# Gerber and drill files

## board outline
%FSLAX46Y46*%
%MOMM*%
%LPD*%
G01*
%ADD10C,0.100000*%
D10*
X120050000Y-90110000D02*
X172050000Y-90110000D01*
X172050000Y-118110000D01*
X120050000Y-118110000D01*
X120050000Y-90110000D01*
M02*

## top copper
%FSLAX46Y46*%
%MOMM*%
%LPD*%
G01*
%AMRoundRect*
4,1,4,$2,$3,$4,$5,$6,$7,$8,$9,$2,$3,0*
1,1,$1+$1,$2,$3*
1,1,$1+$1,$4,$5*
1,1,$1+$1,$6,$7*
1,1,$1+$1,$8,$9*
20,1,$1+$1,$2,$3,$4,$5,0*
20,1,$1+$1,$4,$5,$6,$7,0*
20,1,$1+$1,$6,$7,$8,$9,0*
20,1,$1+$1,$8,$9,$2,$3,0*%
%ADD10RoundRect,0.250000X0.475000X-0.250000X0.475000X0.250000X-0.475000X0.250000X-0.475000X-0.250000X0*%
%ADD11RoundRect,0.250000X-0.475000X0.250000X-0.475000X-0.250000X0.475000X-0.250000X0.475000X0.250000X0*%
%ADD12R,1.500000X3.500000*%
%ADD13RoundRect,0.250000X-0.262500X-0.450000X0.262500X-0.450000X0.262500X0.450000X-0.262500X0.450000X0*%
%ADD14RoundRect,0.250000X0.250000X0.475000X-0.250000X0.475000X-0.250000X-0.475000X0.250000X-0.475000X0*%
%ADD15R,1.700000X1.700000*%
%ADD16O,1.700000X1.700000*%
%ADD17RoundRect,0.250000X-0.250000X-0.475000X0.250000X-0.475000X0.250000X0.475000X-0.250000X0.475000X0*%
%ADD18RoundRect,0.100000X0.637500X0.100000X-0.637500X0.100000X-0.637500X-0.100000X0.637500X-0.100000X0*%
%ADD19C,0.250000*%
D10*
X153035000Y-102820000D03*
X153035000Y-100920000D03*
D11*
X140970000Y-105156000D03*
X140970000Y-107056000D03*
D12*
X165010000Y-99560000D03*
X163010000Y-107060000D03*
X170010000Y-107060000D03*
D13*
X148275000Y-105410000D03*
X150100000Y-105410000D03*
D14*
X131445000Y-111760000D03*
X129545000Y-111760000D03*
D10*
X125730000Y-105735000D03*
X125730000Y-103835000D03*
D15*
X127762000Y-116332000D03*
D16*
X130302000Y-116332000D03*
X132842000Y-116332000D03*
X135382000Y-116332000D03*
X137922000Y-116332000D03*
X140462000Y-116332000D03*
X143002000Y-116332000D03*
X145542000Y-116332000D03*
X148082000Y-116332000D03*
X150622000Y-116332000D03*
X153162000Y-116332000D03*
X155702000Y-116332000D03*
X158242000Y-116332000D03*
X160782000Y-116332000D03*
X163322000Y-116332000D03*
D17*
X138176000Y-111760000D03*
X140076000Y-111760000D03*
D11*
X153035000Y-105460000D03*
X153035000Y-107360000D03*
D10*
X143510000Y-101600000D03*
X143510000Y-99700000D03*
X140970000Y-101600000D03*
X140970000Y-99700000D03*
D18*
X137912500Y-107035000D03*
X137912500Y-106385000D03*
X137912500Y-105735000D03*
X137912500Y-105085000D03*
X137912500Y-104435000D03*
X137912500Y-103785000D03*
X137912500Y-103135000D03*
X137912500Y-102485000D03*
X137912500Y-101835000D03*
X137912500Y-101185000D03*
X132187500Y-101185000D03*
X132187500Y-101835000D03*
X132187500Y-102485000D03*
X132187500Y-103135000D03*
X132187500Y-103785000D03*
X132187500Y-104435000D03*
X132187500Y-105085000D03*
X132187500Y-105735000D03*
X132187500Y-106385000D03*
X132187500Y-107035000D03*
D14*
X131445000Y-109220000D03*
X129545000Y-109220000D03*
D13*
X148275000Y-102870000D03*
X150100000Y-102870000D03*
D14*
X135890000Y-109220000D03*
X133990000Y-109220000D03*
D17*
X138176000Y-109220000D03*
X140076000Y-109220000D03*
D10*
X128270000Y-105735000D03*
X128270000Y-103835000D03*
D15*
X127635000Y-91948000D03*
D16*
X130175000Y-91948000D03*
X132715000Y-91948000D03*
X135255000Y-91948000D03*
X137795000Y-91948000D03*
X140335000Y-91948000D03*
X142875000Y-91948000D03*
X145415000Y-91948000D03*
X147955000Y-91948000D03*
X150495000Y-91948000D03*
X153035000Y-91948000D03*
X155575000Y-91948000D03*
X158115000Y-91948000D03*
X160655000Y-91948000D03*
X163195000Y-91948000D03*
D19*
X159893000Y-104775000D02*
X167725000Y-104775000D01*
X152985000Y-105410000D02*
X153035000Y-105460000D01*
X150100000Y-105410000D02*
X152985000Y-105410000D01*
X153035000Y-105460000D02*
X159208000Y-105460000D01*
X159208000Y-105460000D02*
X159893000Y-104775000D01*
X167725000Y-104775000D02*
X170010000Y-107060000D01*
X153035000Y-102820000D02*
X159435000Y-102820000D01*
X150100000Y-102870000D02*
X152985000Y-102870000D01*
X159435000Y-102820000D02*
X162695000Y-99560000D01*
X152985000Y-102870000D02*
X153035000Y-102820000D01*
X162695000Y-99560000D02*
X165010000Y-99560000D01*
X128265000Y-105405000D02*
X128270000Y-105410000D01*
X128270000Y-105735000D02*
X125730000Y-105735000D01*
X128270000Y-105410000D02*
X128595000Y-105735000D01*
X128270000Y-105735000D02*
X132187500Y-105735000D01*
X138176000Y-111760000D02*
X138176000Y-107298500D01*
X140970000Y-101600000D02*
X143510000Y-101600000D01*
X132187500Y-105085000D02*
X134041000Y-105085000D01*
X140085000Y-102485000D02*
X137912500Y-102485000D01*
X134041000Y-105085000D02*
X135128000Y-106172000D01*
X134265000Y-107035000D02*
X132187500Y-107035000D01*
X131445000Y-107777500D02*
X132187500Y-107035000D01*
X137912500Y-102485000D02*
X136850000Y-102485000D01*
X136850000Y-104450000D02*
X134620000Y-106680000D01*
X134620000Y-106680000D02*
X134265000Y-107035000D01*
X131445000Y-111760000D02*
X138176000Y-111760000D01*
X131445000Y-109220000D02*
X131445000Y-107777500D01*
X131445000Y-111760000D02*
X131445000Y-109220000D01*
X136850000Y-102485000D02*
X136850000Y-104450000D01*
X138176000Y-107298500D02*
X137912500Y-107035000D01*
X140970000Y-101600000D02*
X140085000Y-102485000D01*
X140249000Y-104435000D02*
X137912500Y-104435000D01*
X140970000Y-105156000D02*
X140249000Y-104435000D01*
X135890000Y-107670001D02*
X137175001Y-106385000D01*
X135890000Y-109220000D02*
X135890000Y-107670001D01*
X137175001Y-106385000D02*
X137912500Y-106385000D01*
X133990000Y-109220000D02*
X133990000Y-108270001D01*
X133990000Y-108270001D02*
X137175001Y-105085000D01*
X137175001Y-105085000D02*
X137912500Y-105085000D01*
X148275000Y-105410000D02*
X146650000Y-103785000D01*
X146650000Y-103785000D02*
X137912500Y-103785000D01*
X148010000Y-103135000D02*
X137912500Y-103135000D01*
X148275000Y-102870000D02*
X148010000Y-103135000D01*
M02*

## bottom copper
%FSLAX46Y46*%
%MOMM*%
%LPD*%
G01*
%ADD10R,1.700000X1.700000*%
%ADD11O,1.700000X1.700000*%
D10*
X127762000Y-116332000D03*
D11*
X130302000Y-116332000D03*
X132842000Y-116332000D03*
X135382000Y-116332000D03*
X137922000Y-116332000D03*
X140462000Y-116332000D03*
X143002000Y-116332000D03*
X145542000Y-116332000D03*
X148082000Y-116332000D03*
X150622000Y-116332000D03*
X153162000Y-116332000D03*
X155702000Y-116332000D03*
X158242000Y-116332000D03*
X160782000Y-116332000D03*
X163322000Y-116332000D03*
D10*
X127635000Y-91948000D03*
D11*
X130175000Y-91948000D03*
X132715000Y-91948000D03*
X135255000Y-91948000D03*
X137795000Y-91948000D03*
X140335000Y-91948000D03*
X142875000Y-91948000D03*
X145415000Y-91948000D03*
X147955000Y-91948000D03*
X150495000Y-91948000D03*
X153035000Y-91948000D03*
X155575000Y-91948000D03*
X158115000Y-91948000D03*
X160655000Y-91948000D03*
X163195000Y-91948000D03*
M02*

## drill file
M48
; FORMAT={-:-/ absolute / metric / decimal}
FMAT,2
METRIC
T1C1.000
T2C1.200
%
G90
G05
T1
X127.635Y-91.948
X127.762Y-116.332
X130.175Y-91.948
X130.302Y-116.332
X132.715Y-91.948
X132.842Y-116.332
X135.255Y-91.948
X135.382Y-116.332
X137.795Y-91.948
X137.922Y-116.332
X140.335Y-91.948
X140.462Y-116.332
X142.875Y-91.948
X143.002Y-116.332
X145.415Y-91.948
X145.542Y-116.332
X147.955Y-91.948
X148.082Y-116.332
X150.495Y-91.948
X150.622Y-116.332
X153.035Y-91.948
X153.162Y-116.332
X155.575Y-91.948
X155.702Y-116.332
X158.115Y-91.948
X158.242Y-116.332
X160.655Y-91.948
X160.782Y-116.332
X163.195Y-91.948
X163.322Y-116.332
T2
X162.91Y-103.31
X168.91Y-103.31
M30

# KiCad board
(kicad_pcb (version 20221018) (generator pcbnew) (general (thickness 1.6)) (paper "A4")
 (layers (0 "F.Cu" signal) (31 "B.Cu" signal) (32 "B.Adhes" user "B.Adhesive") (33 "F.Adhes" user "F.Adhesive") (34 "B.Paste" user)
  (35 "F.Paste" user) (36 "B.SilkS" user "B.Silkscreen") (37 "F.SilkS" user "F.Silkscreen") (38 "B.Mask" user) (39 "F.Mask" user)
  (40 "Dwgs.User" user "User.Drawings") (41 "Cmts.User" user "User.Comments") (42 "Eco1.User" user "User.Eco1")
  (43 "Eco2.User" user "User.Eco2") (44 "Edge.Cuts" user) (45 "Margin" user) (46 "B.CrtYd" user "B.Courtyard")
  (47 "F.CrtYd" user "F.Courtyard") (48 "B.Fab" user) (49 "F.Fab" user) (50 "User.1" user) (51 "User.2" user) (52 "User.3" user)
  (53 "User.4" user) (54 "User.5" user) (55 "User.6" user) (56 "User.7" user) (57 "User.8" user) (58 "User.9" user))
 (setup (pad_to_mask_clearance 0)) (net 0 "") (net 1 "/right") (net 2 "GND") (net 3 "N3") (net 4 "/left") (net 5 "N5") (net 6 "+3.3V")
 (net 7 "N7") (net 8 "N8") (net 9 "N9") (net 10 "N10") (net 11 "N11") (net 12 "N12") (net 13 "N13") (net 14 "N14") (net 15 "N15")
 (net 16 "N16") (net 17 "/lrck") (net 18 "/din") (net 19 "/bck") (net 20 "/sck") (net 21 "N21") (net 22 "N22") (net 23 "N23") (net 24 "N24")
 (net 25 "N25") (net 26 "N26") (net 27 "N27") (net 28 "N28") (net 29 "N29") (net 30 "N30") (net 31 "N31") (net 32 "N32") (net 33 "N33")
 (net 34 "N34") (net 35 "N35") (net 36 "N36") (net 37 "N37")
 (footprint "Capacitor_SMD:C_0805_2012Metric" (layer "F.Cu") (at 153.035 101.87 90)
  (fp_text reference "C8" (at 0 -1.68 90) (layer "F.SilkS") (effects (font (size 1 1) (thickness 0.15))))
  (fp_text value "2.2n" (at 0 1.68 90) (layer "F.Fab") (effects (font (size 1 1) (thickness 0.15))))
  (pad "1" smd roundrect (at -0.95 0 90) (size 1 1.45) (layers "F.Cu" "F.Paste" "F.Mask") (roundrect_rratio 0.25) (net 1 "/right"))
  (pad "2" smd roundrect (at 0.95 0 90) (size 1 1.45) (layers "F.Cu" "F.Paste" "F.Mask") (roundrect_rratio 0.25) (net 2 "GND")))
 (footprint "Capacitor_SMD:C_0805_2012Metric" (layer "F.Cu") (at 140.97 106.106 -90)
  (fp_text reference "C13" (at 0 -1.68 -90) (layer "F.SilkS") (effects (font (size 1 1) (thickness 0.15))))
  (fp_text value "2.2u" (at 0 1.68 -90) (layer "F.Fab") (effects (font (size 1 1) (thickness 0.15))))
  (pad "1" smd roundrect (at -0.95 0 270) (size 1 1.45) (layers "F.Cu" "F.Paste" "F.Mask") (roundrect_rratio 0.25) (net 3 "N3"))
  (pad "2" smd roundrect (at 0.95 0 270) (size 1 1.45) (layers "F.Cu" "F.Paste" "F.Mask") (roundrect_rratio 0.25) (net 2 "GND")))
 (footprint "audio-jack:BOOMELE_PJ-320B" (layer "F.Cu") (at 165.91 103.31)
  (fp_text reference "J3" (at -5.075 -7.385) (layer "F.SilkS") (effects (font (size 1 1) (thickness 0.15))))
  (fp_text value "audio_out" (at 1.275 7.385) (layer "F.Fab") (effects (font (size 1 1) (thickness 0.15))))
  (pad "" np_thru_hole circle (at -3 0) (size 1.2 1.2) (drill 1.2) (layers "*.Cu" "*.Mask"))
  (pad "" np_thru_hole circle (at 3 0) (size 1.2 1.2) (drill 1.2) (layers "*.Cu" "*.Mask"))
  (pad "R" smd rect (at -0.9 -3.75) (size 1.5 3.5) (layers "F.Cu" "F.Paste" "F.Mask") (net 1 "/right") (solder_mask_margin 0.102))
  (pad "S" smd rect (at -2.9 3.75) (size 1.5 3.5) (layers "F.Cu" "F.Paste" "F.Mask") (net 2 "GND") (solder_mask_margin 0.102))
  (pad "T" smd rect (at 4.1 3.75) (size 1.5 3.5) (layers "F.Cu" "F.Paste" "F.Mask") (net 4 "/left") (solder_mask_margin 0.102)))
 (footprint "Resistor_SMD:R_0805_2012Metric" (layer "F.Cu") (at 149.1875 105.41)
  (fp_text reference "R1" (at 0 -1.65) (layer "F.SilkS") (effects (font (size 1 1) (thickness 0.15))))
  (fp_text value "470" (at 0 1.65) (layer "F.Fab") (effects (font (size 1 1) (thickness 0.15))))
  (pad "1" smd roundrect (at -0.9125 0) (size 1.025 1.4) (layers "F.Cu" "F.Paste" "F.Mask") (roundrect_rratio 0.243902) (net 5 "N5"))
  (pad "2" smd roundrect (at 0.9125 0) (size 1.025 1.4) (layers "F.Cu" "F.Paste" "F.Mask") (roundrect_rratio 0.243902) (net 4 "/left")))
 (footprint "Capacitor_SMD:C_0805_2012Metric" (layer "F.Cu") (at 130.495 111.76 180)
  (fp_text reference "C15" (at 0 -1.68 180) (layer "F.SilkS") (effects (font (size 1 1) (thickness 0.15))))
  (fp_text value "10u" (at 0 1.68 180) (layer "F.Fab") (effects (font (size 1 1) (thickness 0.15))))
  (pad "1" smd roundrect (at -0.95 0 180) (size 1 1.45) (layers "F.Cu" "F.Paste" "F.Mask") (roundrect_rratio 0.25) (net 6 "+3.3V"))
  (pad "2" smd roundrect (at 0.95 0 180) (size 1 1.45) (layers "F.Cu" "F.Paste" "F.Mask") (roundrect_rratio 0.25) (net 2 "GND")))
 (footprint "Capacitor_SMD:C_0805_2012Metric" (layer "F.Cu") (at 125.73 104.785 90)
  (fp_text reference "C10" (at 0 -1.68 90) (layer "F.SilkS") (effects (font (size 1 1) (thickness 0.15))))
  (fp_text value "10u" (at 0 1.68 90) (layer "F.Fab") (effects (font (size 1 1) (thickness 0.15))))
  (pad "1" smd roundrect (at -0.95 0 90) (size 1 1.45) (layers "F.Cu" "F.Paste" "F.Mask") (roundrect_rratio 0.25) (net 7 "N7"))
  (pad "2" smd roundrect (at 0.95 0 90) (size 1 1.45) (layers "F.Cu" "F.Paste" "F.Mask") (roundrect_rratio 0.25) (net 2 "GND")))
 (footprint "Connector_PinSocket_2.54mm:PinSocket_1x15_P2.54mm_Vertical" (layer "F.Cu") (at 127.762 116.332 90)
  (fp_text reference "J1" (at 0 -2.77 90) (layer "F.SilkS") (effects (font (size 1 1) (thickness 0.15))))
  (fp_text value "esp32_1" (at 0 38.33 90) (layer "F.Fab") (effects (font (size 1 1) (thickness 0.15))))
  (pad "1" thru_hole rect (at 0 0 90) (size 1.7 1.7) (drill 1) (layers "*.Cu" "*.Mask") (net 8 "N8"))
  (pad "2" thru_hole oval (at 0 2.54 90) (size 1.7 1.7) (drill 1) (layers "*.Cu" "*.Mask") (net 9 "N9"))
  (pad "3" thru_hole oval (at 0 5.08 90) (size 1.7 1.7) (drill 1) (layers "*.Cu" "*.Mask") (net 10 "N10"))
  (pad "4" thru_hole oval (at 0 7.62 90) (size 1.7 1.7) (drill 1) (layers "*.Cu" "*.Mask") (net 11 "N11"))
  (pad "5" thru_hole oval (at 0 10.16 90) (size 1.7 1.7) (drill 1) (layers "*.Cu" "*.Mask") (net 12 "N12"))
  (pad "6" thru_hole oval (at 0 12.7 90) (size 1.7 1.7) (drill 1) (layers "*.Cu" "*.Mask") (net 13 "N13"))
  (pad "7" thru_hole oval (at 0 15.24 90) (size 1.7 1.7) (drill 1) (layers "*.Cu" "*.Mask") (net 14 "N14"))
  (pad "8" thru_hole oval (at 0 17.78 90) (size 1.7 1.7) (drill 1) (layers "*.Cu" "*.Mask") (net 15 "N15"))
  (pad "9" thru_hole oval (at 0 20.32 90) (size 1.7 1.7) (drill 1) (layers "*.Cu" "*.Mask") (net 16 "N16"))
  (pad "10" thru_hole oval (at 0 22.86 90) (size 1.7 1.7) (drill 1) (layers "*.Cu" "*.Mask") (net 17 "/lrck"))
  (pad "11" thru_hole oval (at 0 25.4 90) (size 1.7 1.7) (drill 1) (layers "*.Cu" "*.Mask") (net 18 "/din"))
  (pad "12" thru_hole oval (at 0 27.94 90) (size 1.7 1.7) (drill 1) (layers "*.Cu" "*.Mask") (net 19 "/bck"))
  (pad "13" thru_hole oval (at 0 30.48 90) (size 1.7 1.7) (drill 1) (layers "*.Cu" "*.Mask") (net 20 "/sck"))
  (pad "14" thru_hole oval (at 0 33.02 90) (size 1.7 1.7) (drill 1) (layers "*.Cu" "*.Mask") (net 2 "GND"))
  (pad "15" thru_hole oval (at 0 35.56 90) (size 1.7 1.7) (drill 1) (layers "*.Cu" "*.Mask") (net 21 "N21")))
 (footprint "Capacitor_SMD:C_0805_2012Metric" (layer "F.Cu") (at 139.126 111.76)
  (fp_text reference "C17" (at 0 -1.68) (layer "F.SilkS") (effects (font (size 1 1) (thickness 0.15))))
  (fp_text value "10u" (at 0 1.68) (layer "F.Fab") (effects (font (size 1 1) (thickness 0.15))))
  (pad "1" smd roundrect (at -0.95 0) (size 1 1.45) (layers "F.Cu" "F.Paste" "F.Mask") (roundrect_rratio 0.25) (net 6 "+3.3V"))
  (pad "2" smd roundrect (at 0.95 0) (size 1 1.45) (layers "F.Cu" "F.Paste" "F.Mask") (roundrect_rratio 0.25) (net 2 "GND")))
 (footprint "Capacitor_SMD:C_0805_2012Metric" (layer "F.Cu") (at 153.035 106.41 -90)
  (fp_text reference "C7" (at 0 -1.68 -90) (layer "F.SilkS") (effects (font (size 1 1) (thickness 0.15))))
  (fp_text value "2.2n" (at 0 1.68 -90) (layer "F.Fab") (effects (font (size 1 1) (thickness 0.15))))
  (pad "1" smd roundrect (at -0.95 0 270) (size 1 1.45) (layers "F.Cu" "F.Paste" "F.Mask") (roundrect_rratio 0.25) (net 4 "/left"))
  (pad "2" smd roundrect (at 0.95 0 270) (size 1 1.45) (layers "F.Cu" "F.Paste" "F.Mask") (roundrect_rratio 0.25) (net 2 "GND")))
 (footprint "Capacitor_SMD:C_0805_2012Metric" (layer "F.Cu") (at 143.51 100.65 90)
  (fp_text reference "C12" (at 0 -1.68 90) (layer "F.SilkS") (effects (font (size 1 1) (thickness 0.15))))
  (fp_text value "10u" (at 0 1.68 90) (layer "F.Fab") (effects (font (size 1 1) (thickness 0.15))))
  (pad "1" smd roundrect (at -0.95 0 90) (size 1 1.45) (layers "F.Cu" "F.Paste" "F.Mask") (roundrect_rratio 0.25) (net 6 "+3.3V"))
  (pad "2" smd roundrect (at 0.95 0 90) (size 1 1.45) (layers "F.Cu" "F.Paste" "F.Mask") (roundrect_rratio 0.25) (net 2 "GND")))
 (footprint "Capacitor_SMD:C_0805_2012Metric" (layer "F.Cu") (at 140.97 100.65 90)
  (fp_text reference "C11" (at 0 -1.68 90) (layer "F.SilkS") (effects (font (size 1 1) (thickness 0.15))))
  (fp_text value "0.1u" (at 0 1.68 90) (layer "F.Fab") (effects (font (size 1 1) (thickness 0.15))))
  (pad "1" smd roundrect (at -0.95 0 90) (size 1 1.45) (layers "F.Cu" "F.Paste" "F.Mask") (roundrect_rratio 0.25) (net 6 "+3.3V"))
  (pad "2" smd roundrect (at 0.95 0 90) (size 1 1.45) (layers "F.Cu" "F.Paste" "F.Mask") (roundrect_rratio 0.25) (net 2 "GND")))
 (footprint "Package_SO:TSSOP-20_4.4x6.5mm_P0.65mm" (layer "F.Cu") (at 135.05 104.11 180)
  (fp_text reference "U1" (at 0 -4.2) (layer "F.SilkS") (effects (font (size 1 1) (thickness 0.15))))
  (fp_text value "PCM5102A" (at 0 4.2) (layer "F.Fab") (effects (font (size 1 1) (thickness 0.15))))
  (pad "1" smd roundrect (at -2.8625 -2.925 180) (size 1.475 0.4) (layers "F.Cu" "F.Paste" "F.Mask") (roundrect_rratio 0.25) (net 6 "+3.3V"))
  (pad "2" smd roundrect (at -2.8625 -2.275 180) (size 1.475 0.4) (layers "F.Cu" "F.Paste" "F.Mask") (roundrect_rratio 0.25) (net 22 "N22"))
  (pad "3" smd roundrect (at -2.8625 -1.625 180) (size 1.475 0.4) (layers "F.Cu" "F.Paste" "F.Mask") (roundrect_rratio 0.25) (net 2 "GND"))
  (pad "4" smd roundrect (at -2.8625 -0.975 180) (size 1.475 0.4) (layers "F.Cu" "F.Paste" "F.Mask") (roundrect_rratio 0.25) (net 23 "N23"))
  (pad "5" smd roundrect (at -2.8625 -0.325 180) (size 1.475 0.4) (layers "F.Cu" "F.Paste" "F.Mask") (roundrect_rratio 0.25) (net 3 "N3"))
  (pad "6" smd roundrect (at -2.8625 0.325 180) (size 1.475 0.4) (layers "F.Cu" "F.Paste" "F.Mask") (roundrect_rratio 0.25) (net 5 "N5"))
  (pad "7" smd roundrect (at -2.8625 0.975 180) (size 1.475 0.4) (layers "F.Cu" "F.Paste" "F.Mask") (roundrect_rratio 0.25) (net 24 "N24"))
  (pad "8" smd roundrect (at -2.8625 1.625 180) (size 1.475 0.4) (layers "F.Cu" "F.Paste" "F.Mask") (roundrect_rratio 0.25) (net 6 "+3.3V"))
  (pad "9" smd roundrect (at -2.8625 2.275 180) (size 1.475 0.4) (layers "F.Cu" "F.Paste" "F.Mask") (roundrect_rratio 0.25) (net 2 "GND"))
  (pad "10" smd roundrect (at -2.8625 2.925 180) (size 1.475 0.4) (layers "F.Cu" "F.Paste" "F.Mask") (roundrect_rratio 0.25) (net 2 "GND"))
  (pad "11" smd roundrect (at 2.8625 2.925 180) (size 1.475 0.4) (layers "F.Cu" "F.Paste" "F.Mask") (roundrect_rratio 0.25) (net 2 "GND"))
  (pad "12" smd roundrect (at 2.8625 2.275 180) (size 1.475 0.4) (layers "F.Cu" "F.Paste" "F.Mask") (roundrect_rratio 0.25) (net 20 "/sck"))
  (pad "13" smd roundrect (at 2.8625 1.625 180) (size 1.475 0.4) (layers "F.Cu" "F.Paste" "F.Mask") (roundrect_rratio 0.25) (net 19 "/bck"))
  (pad "14" smd roundrect (at 2.8625 0.975 180) (size 1.475 0.4) (layers "F.Cu" "F.Paste" "F.Mask") (roundrect_rratio 0.25) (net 18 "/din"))
  (pad "15" smd roundrect (at 2.8625 0.325 180) (size 1.475 0.4) (layers "F.Cu" "F.Paste" "F.Mask") (roundrect_rratio 0.25) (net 17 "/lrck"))
  (pad "16" smd roundrect (at 2.8625 -0.325 180) (size 1.475 0.4) (layers "F.Cu" "F.Paste" "F.Mask") (roundrect_rratio 0.25) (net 2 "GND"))
  (pad "17" smd roundrect (at 2.8625 -0.975 180) (size 1.475 0.4) (layers "F.Cu" "F.Paste" "F.Mask") (roundrect_rratio 0.25) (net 6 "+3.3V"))
  (pad "18" smd roundrect (at 2.8625 -1.625 180) (size 1.475 0.4) (layers "F.Cu" "F.Paste" "F.Mask") (roundrect_rratio 0.25) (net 7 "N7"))
  (pad "19" smd roundrect (at 2.8625 -2.275 180) (size 1.475 0.4) (layers "F.Cu" "F.Paste" "F.Mask") (roundrect_rratio 0.25) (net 2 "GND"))
  (pad "20" smd roundrect (at 2.8625 -2.925 180) (size 1.475 0.4) (layers "F.Cu" "F.Paste" "F.Mask") (roundrect_rratio 0.25) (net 6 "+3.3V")))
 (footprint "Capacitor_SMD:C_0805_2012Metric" (layer "F.Cu") (at 130.495 109.22 180)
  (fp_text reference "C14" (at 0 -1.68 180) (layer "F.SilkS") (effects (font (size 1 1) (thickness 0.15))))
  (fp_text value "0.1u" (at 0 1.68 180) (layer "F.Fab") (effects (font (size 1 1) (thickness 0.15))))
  (pad "1" smd roundrect (at -0.95 0 180) (size 1 1.45) (layers "F.Cu" "F.Paste" "F.Mask") (roundrect_rratio 0.25) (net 6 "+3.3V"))
  (pad "2" smd roundrect (at 0.95 0 180) (size 1 1.45) (layers "F.Cu" "F.Paste" "F.Mask") (roundrect_rratio 0.25) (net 2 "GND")))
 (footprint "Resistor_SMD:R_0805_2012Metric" (layer "F.Cu") (at 149.1875 102.87)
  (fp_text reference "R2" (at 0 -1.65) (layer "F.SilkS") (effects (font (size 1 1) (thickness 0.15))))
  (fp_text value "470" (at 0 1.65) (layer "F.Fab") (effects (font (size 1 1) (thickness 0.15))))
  (pad "1" smd roundrect (at -0.9125 0) (size 1.025 1.4) (layers "F.Cu" "F.Paste" "F.Mask") (roundrect_rratio 0.243902) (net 24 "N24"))
  (pad "2" smd roundrect (at 0.9125 0) (size 1.025 1.4) (layers "F.Cu" "F.Paste" "F.Mask") (roundrect_rratio 0.243902) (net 1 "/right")))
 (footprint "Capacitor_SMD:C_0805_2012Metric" (layer "F.Cu") (at 134.94 109.22 180)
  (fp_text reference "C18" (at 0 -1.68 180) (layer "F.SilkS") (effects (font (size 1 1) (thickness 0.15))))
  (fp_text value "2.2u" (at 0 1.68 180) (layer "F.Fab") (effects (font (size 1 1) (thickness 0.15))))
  (pad "1" smd roundrect (at -0.95 0 180) (size 1 1.45) (layers "F.Cu" "F.Paste" "F.Mask") (roundrect_rratio 0.25) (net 22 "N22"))
  (pad "2" smd roundrect (at 0.95 0 180) (size 1 1.45) (layers "F.Cu" "F.Paste" "F.Mask") (roundrect_rratio 0.25) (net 23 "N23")))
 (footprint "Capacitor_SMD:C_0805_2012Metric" (layer "F.Cu") (at 139.126 109.22)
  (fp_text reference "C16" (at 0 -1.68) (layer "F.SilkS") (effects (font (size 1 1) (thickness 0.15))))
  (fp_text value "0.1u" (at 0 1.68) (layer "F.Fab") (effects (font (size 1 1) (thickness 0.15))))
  (pad "1" smd roundrect (at -0.95 0) (size 1 1.45) (layers "F.Cu" "F.Paste" "F.Mask") (roundrect_rratio 0.25) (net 6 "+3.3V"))
  (pad "2" smd roundrect (at 0.95 0) (size 1 1.45) (layers "F.Cu" "F.Paste" "F.Mask") (roundrect_rratio 0.25) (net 2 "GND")))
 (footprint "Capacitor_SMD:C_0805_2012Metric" (layer "F.Cu") (at 128.27 104.785 90)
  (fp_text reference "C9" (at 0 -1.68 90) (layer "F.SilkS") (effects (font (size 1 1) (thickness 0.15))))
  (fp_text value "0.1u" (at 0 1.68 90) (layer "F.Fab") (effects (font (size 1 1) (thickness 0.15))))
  (pad "1" smd roundrect (at -0.95 0 90) (size 1 1.45) (layers "F.Cu" "F.Paste" "F.Mask") (roundrect_rratio 0.25) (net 7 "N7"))
  (pad "2" smd roundrect (at 0.95 0 90) (size 1 1.45) (layers "F.Cu" "F.Paste" "F.Mask") (roundrect_rratio 0.25) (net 2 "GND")))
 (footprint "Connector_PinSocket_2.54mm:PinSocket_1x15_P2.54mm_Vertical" (layer "F.Cu") (at 127.635 91.948 90)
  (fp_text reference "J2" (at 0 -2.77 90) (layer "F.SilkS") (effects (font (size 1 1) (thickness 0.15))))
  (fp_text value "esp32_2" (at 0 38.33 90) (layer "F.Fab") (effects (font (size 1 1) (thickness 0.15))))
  (pad "1" thru_hole rect (at 0 0 90) (size 1.7 1.7) (drill 1) (layers "*.Cu" "*.Mask") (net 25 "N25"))
  (pad "2" thru_hole oval (at 0 2.54 90) (size 1.7 1.7) (drill 1) (layers "*.Cu" "*.Mask") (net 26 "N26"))
  (pad "3" thru_hole oval (at 0 5.08 90) (size 1.7 1.7) (drill 1) (layers "*.Cu" "*.Mask") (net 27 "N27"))
  (pad "4" thru_hole oval (at 0 7.62 90) (size 1.7 1.7) (drill 1) (layers "*.Cu" "*.Mask") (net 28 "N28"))
  (pad "5" thru_hole oval (at 0 10.16 90) (size 1.7 1.7) (drill 1) (layers "*.Cu" "*.Mask") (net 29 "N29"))
  (pad "6" thru_hole oval (at 0 12.7 90) (size 1.7 1.7) (drill 1) (layers "*.Cu" "*.Mask") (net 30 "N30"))
  (pad "7" thru_hole oval (at 0 15.24 90) (size 1.7 1.7) (drill 1) (layers "*.Cu" "*.Mask") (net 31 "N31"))
  (pad "8" thru_hole oval (at 0 17.78 90) (size 1.7 1.7) (drill 1) (layers "*.Cu" "*.Mask") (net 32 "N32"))
  (pad "9" thru_hole oval (at 0 20.32 90) (size 1.7 1.7) (drill 1) (layers "*.Cu" "*.Mask") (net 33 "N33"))
  (pad "10" thru_hole oval (at 0 22.86 90) (size 1.7 1.7) (drill 1) (layers "*.Cu" "*.Mask") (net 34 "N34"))
  (pad "11" thru_hole oval (at 0 25.4 90) (size 1.7 1.7) (drill 1) (layers "*.Cu" "*.Mask") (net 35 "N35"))
  (pad "12" thru_hole oval (at 0 27.94 90) (size 1.7 1.7) (drill 1) (layers "*.Cu" "*.Mask") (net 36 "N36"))
  (pad "13" thru_hole oval (at 0 30.48 90) (size 1.7 1.7) (drill 1) (layers "*.Cu" "*.Mask") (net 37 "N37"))
  (pad "14" thru_hole oval (at 0 33.02 90) (size 1.7 1.7) (drill 1) (layers "*.Cu" "*.Mask") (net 2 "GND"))
  (pad "15" thru_hole oval (at 0 35.56 90) (size 1.7 1.7) (drill 1) (layers "*.Cu" "*.Mask") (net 6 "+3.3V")))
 (gr_rect (start 120.05 90.11) (end 172.05 118.11) (stroke (width 0.1) (type default)) (fill none) (layer "Edge.Cuts"))
 (segment (start 159.893 104.775) (end 167.725 104.775) (width 0.25) (layer "F.Cu") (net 4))
 (segment (start 152.985 105.41) (end 153.035 105.46) (width 0.25) (layer "F.Cu") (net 4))
 (segment (start 150.1 105.41) (end 152.985 105.41) (width 0.25) (layer "F.Cu") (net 4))
 (segment (start 153.035 105.46) (end 159.208 105.46) (width 0.25) (layer "F.Cu") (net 4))
 (segment (start 159.208 105.46) (end 159.893 104.775) (width 0.25) (layer "F.Cu") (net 4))
 (segment (start 167.725 104.775) (end 170.01 107.06) (width 0.25) (layer "F.Cu") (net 4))
 (segment (start 153.035 102.82) (end 159.435 102.82) (width 0.25) (layer "F.Cu") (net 1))
 (segment (start 150.1 102.87) (end 152.985 102.87) (width 0.25) (layer "F.Cu") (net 1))
 (segment (start 159.435 102.82) (end 162.695 99.56) (width 0.25) (layer "F.Cu") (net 1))
 (segment (start 152.985 102.87) (end 153.035 102.82) (width 0.25) (layer "F.Cu") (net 1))
 (segment (start 162.695 99.56) (end 165.01 99.56) (width 0.25) (layer "F.Cu") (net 1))
 (segment (start 128.265 105.405) (end 128.27 105.41) (width 0.25) (layer "F.Cu") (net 7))
 (segment (start 128.27 105.735) (end 125.73 105.735) (width 0.25) (layer "F.Cu") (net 7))
 (segment (start 128.27 105.41) (end 128.595 105.735) (width 0.25) (layer "F.Cu") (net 7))
 (segment (start 128.27 105.735) (end 132.1875 105.735) (width 0.25) (layer "F.Cu") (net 7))
 (segment (start 138.176 111.76) (end 138.176 107.2985) (width 0.25) (layer "F.Cu") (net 6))
 (segment (start 140.97 101.6) (end 143.51 101.6) (width 0.25) (layer "F.Cu") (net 6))
 (segment (start 132.1875 105.085) (end 134.041 105.085) (width 0.25) (layer "F.Cu") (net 6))
 (segment (start 140.085 102.485) (end 137.9125 102.485) (width 0.25) (layer "F.Cu") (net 6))
 (segment (start 134.041 105.085) (end 135.128 106.172) (width 0.25) (layer "F.Cu") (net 6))
 (segment (start 134.265 107.035) (end 132.1875 107.035) (width 0.25) (layer "F.Cu") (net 6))
 (segment (start 131.445 107.7775) (end 132.1875 107.035) (width 0.25) (layer "F.Cu") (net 6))
 (segment (start 137.9125 102.485) (end 136.85 102.485) (width 0.25) (layer "F.Cu") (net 6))
 (segment (start 136.85 104.45) (end 134.62 106.68) (width 0.25) (layer "F.Cu") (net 6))
 (segment (start 134.62 106.68) (end 134.265 107.035) (width 0.25) (layer "F.Cu") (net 6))
 (segment (start 131.445 111.76) (end 138.176 111.76) (width 0.25) (layer "F.Cu") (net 6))
 (segment (start 131.445 109.22) (end 131.445 107.7775) (width 0.25) (layer "F.Cu") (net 6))
 (segment (start 131.445 111.76) (end 131.445 109.22) (width 0.25) (layer "F.Cu") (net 6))
 (segment (start 136.85 102.485) (end 136.85 104.45) (width 0.25) (layer "F.Cu") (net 6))
 (segment (start 138.176 107.2985) (end 137.9125 107.035) (width 0.25) (layer "F.Cu") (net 6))
 (segment (start 140.97 101.6) (end 140.085 102.485) (width 0.25) (layer "F.Cu") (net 6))
 (segment (start 140.249 104.435) (end 137.9125 104.435) (width 0.25) (layer "F.Cu") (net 3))
 (segment (start 140.97 105.156) (end 140.249 104.435) (width 0.25) (layer "F.Cu") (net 3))
 (segment (start 135.89 107.670001) (end 137.175001 106.385) (width 0.25) (layer "F.Cu") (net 22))
 (segment (start 135.89 109.22) (end 135.89 107.670001) (width 0.25) (layer "F.Cu") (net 22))
 (segment (start 137.175001 106.385) (end 137.9125 106.385) (width 0.25) (layer "F.Cu") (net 22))
 (segment (start 133.99 109.22) (end 133.99 108.270001) (width 0.25) (layer "F.Cu") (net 23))
 (segment (start 133.99 108.270001) (end 137.175001 105.085) (width 0.25) (layer "F.Cu") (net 23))
 (segment (start 137.175001 105.085) (end 137.9125 105.085) (width 0.25) (layer "F.Cu") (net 23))
 (segment (start 148.275 105.41) (end 146.65 103.785) (width 0.25) (layer "F.Cu") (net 5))
 (segment (start 146.65 103.785) (end 137.9125 103.785) (width 0.25) (layer "F.Cu") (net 5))
 (segment (start 148.01 103.135) (end 137.9125 103.135) (width 0.25) (layer "F.Cu") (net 24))
 (segment (start 148.275 102.87) (end 148.01 103.135) (width 0.25) (layer "F.Cu") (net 24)))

